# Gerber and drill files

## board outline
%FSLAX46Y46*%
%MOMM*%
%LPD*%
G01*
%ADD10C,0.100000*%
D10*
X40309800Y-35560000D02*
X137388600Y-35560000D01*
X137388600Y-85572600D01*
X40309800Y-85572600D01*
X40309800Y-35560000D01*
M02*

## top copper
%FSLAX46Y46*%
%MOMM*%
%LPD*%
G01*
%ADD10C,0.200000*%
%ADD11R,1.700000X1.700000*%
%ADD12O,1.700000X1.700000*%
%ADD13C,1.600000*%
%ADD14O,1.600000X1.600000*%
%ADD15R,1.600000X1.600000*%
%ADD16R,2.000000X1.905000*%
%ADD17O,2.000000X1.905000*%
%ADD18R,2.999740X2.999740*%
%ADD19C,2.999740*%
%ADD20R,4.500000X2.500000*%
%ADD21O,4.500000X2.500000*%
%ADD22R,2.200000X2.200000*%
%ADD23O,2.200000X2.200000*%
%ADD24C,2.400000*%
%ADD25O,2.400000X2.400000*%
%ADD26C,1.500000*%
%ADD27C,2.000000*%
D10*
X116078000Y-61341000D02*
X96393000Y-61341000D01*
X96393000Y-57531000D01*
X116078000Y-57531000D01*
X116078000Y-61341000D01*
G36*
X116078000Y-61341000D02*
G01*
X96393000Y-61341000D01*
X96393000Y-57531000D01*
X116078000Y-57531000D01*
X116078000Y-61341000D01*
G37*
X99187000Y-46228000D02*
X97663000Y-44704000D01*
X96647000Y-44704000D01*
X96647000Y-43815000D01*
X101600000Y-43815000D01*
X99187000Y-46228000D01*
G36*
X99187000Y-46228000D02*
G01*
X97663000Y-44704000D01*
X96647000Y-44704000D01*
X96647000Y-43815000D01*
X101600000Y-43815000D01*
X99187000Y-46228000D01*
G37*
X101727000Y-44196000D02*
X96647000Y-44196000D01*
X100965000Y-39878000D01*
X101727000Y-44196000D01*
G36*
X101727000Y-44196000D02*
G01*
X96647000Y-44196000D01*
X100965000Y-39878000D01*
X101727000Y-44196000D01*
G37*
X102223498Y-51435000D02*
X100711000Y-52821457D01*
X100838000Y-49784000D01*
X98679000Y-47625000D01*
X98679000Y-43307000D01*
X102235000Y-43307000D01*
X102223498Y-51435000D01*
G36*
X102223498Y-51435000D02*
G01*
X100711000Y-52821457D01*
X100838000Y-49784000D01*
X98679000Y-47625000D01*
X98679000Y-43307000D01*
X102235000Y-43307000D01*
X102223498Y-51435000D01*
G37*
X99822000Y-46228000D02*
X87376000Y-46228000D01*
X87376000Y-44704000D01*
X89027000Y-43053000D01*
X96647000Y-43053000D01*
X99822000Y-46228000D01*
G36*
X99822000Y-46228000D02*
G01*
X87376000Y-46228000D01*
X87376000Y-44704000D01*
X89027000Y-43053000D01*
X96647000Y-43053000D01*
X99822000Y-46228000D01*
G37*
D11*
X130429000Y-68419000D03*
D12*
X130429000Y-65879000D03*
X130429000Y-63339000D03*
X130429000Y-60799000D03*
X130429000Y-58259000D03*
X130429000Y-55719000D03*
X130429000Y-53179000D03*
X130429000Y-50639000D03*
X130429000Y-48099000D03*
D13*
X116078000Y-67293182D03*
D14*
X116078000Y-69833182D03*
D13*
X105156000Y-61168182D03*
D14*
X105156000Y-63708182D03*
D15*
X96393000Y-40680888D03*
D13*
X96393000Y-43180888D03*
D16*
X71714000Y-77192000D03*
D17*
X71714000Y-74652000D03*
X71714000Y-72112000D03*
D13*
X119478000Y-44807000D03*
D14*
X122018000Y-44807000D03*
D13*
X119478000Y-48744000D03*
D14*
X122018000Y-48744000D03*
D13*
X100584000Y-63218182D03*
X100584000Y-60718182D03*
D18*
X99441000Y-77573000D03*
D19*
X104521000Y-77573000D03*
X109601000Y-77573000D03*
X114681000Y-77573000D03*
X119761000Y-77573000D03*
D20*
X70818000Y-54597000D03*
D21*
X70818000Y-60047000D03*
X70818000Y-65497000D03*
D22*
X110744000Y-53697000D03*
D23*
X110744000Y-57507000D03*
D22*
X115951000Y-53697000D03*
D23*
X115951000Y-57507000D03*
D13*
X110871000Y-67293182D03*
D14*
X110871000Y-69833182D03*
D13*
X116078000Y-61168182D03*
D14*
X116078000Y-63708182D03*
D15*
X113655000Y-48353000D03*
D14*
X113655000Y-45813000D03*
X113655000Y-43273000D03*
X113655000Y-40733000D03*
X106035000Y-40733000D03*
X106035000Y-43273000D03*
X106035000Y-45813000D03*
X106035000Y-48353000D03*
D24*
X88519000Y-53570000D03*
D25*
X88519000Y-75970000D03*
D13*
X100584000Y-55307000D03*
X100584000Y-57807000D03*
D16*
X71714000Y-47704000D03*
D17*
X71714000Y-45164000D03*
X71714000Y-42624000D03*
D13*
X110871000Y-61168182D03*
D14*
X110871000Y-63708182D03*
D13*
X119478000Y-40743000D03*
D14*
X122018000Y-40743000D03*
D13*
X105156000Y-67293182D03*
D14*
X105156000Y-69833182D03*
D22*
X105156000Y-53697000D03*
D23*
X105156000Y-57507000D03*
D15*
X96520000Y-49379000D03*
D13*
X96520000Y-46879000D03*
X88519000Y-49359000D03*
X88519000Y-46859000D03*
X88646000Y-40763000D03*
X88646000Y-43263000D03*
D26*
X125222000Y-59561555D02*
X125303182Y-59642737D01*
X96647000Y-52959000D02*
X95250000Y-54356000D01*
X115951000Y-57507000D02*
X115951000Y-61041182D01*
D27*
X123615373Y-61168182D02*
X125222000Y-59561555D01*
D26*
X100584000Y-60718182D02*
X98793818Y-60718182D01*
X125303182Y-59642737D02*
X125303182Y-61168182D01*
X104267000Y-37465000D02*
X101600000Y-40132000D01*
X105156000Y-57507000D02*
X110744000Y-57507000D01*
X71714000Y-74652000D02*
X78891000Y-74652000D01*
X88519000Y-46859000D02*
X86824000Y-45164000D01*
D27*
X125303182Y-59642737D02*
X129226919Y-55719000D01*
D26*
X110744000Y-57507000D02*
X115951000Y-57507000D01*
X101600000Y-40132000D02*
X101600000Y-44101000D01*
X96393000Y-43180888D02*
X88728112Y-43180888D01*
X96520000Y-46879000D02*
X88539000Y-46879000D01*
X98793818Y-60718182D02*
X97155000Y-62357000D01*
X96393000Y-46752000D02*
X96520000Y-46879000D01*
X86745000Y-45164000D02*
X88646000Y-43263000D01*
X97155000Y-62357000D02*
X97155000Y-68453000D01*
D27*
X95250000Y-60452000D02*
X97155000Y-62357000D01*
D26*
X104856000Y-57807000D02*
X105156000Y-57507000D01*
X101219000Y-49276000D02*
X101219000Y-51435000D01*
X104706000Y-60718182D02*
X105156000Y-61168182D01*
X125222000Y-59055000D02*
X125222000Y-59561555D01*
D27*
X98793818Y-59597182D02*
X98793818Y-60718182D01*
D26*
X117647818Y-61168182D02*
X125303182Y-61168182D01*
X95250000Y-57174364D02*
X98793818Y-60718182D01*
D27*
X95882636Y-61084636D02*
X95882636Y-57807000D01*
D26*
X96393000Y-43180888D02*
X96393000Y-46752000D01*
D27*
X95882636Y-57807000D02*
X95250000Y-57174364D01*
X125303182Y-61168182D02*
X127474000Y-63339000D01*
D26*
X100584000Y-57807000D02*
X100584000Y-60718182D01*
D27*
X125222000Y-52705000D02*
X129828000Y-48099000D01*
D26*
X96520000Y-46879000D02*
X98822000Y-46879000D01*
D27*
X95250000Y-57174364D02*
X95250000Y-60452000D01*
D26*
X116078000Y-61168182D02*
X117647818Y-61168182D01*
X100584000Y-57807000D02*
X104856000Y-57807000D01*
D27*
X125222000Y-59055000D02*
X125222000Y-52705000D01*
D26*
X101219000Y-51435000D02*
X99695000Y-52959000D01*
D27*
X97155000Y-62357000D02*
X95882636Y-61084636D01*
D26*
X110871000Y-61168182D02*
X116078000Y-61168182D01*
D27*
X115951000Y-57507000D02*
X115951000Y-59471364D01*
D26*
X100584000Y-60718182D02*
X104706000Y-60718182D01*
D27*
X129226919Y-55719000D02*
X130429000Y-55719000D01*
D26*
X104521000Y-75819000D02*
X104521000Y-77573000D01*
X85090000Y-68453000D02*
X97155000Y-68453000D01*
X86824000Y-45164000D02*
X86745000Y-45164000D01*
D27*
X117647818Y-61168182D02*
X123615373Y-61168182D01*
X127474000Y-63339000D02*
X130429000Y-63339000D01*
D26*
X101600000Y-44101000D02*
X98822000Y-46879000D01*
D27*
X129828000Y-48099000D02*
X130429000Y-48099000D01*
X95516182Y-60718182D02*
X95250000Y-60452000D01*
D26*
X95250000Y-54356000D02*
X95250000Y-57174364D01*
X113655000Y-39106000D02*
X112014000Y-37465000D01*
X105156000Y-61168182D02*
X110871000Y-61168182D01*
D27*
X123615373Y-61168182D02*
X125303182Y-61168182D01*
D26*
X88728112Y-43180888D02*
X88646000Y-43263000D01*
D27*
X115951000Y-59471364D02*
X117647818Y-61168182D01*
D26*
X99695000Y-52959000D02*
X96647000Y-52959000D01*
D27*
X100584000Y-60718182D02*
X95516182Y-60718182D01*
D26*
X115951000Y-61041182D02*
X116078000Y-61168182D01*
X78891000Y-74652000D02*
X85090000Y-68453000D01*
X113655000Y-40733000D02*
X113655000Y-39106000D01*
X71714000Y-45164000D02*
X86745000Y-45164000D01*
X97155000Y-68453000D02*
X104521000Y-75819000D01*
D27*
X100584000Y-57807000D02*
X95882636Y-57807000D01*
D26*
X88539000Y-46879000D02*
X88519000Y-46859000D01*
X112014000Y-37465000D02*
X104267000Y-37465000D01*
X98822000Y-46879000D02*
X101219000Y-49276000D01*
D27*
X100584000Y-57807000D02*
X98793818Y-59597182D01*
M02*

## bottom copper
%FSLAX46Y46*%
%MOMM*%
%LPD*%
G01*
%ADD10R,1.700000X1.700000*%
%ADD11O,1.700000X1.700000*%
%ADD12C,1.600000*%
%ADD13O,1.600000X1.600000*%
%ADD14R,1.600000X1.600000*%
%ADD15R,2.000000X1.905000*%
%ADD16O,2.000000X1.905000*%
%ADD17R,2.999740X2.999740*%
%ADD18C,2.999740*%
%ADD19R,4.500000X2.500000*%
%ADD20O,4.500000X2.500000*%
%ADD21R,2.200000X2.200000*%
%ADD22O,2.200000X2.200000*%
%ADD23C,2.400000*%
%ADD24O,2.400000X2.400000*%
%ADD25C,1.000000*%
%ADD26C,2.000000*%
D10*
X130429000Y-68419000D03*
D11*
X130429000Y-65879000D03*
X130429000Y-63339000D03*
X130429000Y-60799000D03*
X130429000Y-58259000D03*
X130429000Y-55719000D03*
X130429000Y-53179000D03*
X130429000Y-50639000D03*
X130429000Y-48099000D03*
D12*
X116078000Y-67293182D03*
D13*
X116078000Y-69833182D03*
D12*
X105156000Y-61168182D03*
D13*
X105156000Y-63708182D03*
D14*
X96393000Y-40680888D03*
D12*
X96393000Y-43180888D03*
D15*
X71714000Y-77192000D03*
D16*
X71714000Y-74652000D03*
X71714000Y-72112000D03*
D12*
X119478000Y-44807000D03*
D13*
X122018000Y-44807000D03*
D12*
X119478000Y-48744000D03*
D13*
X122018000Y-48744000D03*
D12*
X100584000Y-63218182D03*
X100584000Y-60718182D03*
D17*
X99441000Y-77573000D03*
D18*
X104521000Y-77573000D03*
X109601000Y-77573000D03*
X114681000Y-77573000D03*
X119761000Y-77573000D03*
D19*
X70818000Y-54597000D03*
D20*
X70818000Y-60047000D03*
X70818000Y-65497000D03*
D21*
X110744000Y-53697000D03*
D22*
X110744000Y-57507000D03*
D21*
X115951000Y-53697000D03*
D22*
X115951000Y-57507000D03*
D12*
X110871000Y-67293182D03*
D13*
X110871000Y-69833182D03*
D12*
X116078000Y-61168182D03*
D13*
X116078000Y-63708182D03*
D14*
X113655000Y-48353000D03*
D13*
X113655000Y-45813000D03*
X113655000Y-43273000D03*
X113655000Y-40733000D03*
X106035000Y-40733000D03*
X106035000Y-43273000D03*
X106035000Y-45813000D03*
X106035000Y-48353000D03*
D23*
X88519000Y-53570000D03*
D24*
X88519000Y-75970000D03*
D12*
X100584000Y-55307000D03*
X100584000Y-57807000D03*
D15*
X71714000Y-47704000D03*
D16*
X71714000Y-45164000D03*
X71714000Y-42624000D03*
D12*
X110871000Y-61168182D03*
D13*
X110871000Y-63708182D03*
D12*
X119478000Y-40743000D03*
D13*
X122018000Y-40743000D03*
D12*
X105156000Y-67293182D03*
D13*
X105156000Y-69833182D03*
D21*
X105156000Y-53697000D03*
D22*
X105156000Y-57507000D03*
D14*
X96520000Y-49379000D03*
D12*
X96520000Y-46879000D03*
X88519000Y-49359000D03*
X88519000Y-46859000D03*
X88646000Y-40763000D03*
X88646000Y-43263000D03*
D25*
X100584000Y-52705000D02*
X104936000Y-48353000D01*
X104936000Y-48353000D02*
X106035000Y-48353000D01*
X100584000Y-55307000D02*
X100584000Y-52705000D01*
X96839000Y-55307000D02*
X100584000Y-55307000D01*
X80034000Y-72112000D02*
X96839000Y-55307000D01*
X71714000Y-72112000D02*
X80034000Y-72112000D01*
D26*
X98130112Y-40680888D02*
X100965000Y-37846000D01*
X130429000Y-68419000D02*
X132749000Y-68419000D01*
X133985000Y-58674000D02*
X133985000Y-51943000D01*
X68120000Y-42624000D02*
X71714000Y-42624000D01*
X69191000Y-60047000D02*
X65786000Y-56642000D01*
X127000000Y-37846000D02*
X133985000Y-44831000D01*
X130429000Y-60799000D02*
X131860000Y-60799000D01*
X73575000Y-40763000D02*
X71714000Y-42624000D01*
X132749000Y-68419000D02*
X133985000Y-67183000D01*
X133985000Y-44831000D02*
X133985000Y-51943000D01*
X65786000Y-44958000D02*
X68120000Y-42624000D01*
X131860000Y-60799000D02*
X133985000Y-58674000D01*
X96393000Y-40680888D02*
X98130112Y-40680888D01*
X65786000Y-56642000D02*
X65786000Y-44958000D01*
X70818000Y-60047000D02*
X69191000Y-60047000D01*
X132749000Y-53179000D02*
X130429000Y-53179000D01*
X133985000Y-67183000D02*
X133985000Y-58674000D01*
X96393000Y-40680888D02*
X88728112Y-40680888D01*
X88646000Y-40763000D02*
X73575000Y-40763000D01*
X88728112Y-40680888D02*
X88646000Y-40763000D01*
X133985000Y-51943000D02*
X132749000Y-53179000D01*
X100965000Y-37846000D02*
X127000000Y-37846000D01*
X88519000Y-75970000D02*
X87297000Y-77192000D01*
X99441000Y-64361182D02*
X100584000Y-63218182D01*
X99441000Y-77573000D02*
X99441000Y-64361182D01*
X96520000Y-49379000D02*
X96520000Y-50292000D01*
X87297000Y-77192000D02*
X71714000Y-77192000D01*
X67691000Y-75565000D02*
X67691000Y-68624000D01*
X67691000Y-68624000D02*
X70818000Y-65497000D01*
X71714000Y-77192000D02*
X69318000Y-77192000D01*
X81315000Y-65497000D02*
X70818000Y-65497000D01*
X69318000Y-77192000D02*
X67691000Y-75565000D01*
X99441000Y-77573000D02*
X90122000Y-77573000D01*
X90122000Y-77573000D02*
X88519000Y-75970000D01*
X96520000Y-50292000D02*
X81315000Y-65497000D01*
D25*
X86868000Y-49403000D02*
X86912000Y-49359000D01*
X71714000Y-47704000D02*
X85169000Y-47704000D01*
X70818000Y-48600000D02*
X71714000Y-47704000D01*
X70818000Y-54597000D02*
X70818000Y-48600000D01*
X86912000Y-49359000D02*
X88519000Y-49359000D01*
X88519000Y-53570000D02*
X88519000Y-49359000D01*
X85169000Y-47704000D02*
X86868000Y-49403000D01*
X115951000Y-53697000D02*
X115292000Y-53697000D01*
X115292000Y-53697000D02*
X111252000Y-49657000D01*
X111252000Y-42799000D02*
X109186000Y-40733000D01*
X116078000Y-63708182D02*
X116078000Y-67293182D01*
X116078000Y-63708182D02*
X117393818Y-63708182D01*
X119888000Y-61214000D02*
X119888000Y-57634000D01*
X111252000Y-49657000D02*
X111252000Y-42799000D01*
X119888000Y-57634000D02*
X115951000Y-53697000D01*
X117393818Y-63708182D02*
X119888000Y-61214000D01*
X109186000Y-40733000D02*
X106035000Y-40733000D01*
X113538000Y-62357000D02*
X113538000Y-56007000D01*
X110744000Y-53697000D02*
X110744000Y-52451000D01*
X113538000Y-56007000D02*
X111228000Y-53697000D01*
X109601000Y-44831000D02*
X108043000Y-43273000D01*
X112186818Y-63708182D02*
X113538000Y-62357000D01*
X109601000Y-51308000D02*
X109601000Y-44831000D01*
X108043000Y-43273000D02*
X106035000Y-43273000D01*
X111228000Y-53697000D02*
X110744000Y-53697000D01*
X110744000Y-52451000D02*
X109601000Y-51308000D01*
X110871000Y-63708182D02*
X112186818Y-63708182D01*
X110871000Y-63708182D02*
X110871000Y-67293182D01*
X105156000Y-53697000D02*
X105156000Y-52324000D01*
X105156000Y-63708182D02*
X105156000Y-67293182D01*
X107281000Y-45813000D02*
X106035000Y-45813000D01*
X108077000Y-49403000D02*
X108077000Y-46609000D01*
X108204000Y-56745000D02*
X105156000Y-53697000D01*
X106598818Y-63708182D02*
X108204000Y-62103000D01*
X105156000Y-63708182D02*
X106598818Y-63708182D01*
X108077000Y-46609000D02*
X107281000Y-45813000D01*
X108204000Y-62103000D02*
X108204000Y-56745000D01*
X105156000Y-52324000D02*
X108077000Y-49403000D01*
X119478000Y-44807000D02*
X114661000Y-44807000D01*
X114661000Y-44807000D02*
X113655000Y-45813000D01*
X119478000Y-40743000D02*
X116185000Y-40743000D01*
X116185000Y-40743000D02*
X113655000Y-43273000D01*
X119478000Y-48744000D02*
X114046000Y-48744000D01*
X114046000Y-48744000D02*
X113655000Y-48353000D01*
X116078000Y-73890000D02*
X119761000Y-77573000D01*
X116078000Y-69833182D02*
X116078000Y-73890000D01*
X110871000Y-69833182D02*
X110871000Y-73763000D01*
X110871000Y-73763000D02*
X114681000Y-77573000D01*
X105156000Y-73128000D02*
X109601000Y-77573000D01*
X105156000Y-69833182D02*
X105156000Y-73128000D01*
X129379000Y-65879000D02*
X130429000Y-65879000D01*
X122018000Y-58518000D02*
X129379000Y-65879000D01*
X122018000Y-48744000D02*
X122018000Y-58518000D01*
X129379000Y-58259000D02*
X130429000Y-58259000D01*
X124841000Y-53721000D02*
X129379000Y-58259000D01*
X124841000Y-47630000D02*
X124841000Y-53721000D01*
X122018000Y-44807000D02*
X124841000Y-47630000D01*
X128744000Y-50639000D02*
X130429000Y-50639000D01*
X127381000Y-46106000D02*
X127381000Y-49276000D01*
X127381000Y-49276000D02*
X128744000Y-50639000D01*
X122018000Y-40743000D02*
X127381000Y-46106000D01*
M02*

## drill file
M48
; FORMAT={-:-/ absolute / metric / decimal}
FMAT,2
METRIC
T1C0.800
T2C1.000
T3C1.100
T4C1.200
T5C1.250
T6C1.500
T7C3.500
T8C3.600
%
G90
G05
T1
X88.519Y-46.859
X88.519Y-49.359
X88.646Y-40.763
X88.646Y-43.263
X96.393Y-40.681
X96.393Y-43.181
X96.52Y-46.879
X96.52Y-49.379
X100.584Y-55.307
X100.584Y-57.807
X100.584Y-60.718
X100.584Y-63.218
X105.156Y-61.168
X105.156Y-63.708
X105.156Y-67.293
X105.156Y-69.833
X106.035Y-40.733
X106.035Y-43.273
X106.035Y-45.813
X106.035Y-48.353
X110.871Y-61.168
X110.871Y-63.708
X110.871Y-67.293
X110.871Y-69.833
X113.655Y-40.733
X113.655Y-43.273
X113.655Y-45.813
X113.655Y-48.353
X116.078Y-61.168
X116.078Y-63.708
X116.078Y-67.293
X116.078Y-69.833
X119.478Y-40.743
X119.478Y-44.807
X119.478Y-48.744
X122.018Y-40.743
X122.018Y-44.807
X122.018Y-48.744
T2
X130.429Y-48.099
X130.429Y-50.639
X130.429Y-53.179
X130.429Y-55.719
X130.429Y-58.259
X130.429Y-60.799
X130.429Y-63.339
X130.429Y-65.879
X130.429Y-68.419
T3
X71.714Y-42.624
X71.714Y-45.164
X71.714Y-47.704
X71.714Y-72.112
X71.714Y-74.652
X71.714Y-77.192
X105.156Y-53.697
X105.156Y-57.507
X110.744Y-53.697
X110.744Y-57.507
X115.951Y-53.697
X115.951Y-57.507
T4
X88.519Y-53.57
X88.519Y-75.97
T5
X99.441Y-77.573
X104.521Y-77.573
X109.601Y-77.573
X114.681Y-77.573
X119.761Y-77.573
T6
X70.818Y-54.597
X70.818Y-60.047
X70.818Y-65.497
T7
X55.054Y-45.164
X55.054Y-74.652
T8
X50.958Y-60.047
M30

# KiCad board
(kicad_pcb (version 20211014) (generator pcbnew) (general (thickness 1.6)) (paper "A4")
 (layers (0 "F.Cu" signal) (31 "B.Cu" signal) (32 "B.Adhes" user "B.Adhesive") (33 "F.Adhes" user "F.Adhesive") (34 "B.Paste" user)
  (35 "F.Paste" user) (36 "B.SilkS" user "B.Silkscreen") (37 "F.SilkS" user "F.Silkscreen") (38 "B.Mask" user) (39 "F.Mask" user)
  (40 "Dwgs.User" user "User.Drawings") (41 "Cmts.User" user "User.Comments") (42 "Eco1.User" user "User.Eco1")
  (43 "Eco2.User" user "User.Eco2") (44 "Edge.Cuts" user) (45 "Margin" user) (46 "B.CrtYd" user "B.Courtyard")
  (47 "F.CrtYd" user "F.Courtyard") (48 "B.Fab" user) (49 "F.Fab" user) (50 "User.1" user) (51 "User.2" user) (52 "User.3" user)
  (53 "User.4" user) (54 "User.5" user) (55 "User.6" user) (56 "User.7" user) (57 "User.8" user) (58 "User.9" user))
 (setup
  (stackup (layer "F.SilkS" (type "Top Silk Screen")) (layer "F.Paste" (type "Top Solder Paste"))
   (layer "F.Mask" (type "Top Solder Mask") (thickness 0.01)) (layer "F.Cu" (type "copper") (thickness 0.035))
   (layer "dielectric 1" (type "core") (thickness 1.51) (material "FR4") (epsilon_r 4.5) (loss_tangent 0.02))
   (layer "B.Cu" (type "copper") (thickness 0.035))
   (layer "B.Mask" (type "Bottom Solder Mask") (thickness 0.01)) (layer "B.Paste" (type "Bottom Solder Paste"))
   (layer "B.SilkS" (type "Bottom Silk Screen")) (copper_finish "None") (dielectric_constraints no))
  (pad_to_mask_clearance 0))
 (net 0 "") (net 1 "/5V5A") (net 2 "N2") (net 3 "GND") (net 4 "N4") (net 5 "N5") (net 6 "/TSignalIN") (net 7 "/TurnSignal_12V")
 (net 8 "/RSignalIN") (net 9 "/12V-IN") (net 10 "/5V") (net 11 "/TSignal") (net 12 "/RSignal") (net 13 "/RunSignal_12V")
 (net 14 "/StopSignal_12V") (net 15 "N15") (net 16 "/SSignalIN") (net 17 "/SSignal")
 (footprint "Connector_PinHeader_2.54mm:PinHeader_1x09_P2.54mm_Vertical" (layer "F.Cu") (at 130.429 68.419 180)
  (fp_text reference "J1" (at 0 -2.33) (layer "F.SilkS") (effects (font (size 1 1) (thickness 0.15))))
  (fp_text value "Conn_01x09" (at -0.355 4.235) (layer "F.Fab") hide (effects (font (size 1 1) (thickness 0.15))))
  (pad "1" thru_hole rect (at 0 0 180) (size 1.7 1.7) (drill 1) (layers *.Cu *.Mask) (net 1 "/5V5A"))
  (pad "2" thru_hole oval (at 0 2.54 180) (size 1.7 1.7) (drill 1) (layers *.Cu *.Mask) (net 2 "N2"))
  (pad "3" thru_hole oval (at 0 5.08 180) (size 1.7 1.7) (drill 1) (layers *.Cu *.Mask) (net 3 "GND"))
  (pad "4" thru_hole oval (at 0 7.62 180) (size 1.7 1.7) (drill 1) (layers *.Cu *.Mask) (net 1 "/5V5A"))
  (pad "5" thru_hole oval (at 0 10.16 180) (size 1.7 1.7) (drill 1) (layers *.Cu *.Mask) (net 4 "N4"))
  (pad "6" thru_hole oval (at 0 12.7 180) (size 1.7 1.7) (drill 1) (layers *.Cu *.Mask) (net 3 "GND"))
  (pad "7" thru_hole oval (at 0 15.24 180) (size 1.7 1.7) (drill 1) (layers *.Cu *.Mask) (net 1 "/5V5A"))
  (pad "8" thru_hole oval (at 0 17.78 180) (size 1.7 1.7) (drill 1) (layers *.Cu *.Mask) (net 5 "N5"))
  (pad "9" thru_hole oval (at 0 20.32 180) (size 1.7 1.7) (drill 1) (layers *.Cu *.Mask) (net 3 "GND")))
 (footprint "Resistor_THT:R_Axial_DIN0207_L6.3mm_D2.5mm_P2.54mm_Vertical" (layer "F.Cu") (at 116.078 67.293182 -90)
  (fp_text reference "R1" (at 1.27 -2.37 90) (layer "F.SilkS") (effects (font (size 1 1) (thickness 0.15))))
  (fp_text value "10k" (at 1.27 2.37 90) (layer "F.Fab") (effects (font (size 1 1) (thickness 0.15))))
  (pad "1" thru_hole circle (at 0 0 270) (size 1.6 1.6) (drill 0.8) (layers *.Cu *.Mask) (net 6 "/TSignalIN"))
  (pad "2" thru_hole oval (at 2.54 0 270) (size 1.6 1.6) (drill 0.8) (layers *.Cu *.Mask) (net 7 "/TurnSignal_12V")))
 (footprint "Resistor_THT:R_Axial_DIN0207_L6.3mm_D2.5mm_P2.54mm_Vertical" (layer "F.Cu") (at 105.156 61.168182 -90)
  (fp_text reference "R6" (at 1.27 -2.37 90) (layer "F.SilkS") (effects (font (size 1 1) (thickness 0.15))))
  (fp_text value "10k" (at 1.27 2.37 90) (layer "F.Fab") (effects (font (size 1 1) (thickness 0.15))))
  (pad "1" thru_hole circle (at 0 0 270) (size 1.6 1.6) (drill 0.8) (layers *.Cu *.Mask) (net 3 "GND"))
  (pad "2" thru_hole oval (at 2.54 0 270) (size 1.6 1.6) (drill 0.8) (layers *.Cu *.Mask) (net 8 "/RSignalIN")))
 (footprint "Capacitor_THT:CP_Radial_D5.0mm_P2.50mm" (layer "F.Cu") (at 96.393 40.680888 -90)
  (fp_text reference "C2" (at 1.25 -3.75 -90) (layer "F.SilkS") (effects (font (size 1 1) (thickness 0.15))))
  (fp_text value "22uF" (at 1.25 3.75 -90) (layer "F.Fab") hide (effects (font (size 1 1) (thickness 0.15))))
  (pad "1" thru_hole rect (at 0 0 270) (size 1.6 1.6) (drill 0.8) (layers *.Cu *.Mask) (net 1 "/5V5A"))
  (pad "2" thru_hole circle (at 2.5 0 270) (size 1.6 1.6) (drill 0.8) (layers *.Cu *.Mask) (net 3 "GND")))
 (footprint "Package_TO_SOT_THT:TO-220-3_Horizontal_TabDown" (layer "F.Cu") (at 71.714 77.192 90)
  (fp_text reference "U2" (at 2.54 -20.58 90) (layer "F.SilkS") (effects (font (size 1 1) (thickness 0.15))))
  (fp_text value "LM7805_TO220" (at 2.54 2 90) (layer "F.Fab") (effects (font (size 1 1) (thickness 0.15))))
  (pad "" np_thru_hole oval (at 2.54 -16.66 90) (size 3.5 3.5) (drill 3.5) (layers *.Cu *.Mask))
  (pad "1" thru_hole rect (at 0 0 90) (size 1.905 2) (drill 1.1) (layers *.Cu *.Mask) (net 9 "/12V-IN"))
  (pad "2" thru_hole oval (at 2.54 0 90) (size 1.905 2) (drill 1.1) (layers *.Cu *.Mask) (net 3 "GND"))
  (pad "3" thru_hole oval (at 5.08 0 90) (size 1.905 2) (drill 1.1) (layers *.Cu *.Mask) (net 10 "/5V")))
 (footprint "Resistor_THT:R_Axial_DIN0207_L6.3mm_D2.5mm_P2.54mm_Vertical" (layer "F.Cu") (at 119.478 44.807)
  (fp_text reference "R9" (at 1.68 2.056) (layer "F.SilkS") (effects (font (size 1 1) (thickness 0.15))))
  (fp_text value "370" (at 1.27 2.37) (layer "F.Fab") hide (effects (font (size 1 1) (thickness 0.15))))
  (pad "1" thru_hole circle (at 0 0) (size 1.6 1.6) (drill 0.8) (layers *.Cu *.Mask) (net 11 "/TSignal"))
  (pad "2" thru_hole oval (at 2.54 0) (size 1.6 1.6) (drill 0.8) (layers *.Cu *.Mask) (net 4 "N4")))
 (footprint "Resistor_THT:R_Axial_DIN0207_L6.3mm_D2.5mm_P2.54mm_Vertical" (layer "F.Cu") (at 119.478 48.744)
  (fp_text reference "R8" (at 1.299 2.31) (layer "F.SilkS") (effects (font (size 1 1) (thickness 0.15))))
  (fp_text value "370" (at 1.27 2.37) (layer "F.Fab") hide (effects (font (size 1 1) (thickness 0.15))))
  (pad "1" thru_hole circle (at 0 0) (size 1.6 1.6) (drill 0.8) (layers *.Cu *.Mask) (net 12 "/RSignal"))
  (pad "2" thru_hole oval (at 2.54 0) (size 1.6 1.6) (drill 0.8) (layers *.Cu *.Mask) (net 2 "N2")))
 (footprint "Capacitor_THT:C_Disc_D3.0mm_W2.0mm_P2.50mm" (layer "F.Cu") (at 100.584 63.218182 90)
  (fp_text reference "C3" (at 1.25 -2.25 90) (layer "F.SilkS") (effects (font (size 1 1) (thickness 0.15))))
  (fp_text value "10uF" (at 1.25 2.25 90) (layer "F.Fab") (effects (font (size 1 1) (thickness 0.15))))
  (pad "1" thru_hole circle (at 0 0 90) (size 1.6 1.6) (drill 0.8) (layers *.Cu *.Mask) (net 9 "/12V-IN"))
  (pad "2" thru_hole circle (at 2.5 0 90) (size 1.6 1.6) (drill 0.8) (layers *.Cu *.Mask) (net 3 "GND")))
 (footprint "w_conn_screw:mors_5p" (layer "F.Cu") (at 109.601 77.573)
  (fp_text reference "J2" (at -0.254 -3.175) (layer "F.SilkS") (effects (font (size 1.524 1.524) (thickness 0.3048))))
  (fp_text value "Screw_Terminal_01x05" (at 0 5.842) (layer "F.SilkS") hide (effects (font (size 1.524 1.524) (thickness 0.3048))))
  (pad "1" thru_hole rect locked (at -10.16 0) (size 2.99974 2.99974) (drill 1.24968) (layers *.Cu *.Mask "F.SilkS") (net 9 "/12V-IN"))
  (pad "2" thru_hole circle locked (at -5.08 0) (size 2.99974 2.99974) (drill 1.24968) (layers *.Cu *.Mask "F.SilkS") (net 3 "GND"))
  (pad "3" thru_hole circle locked (at 0 0) (size 2.99974 2.99974) (drill 1.24968) (layers *.Cu *.Mask "F.SilkS") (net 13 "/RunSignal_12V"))
  (pad "4" thru_hole circle locked (at 5.08 0) (size 2.99974 2.99974) (drill 1.24968) (layers *.Cu *.Mask "F.SilkS")
   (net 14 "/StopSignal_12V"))
  (pad "5" thru_hole circle locked (at 10.16 0) (size 2.99974 2.99974) (drill 1.24968) (layers *.Cu *.Mask "F.SilkS")
   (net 7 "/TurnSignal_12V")))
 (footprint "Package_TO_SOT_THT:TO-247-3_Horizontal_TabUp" (layer "F.Cu") (at 70.818 54.597 -90)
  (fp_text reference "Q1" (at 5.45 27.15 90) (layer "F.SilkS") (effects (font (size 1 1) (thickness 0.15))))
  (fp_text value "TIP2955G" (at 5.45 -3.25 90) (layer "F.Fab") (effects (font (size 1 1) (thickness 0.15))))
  (pad "" np_thru_hole oval (at 5.45 19.86 270) (size 3.6 3.6) (drill 3.6) (layers *.Cu *.Mask))
  (pad "1" thru_hole rect (at 0 0 270) (size 2.5 4.5) (drill 1.5) (layers *.Cu *.Mask) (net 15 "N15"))
  (pad "2" thru_hole oval (at 5.45 0 270) (size 2.5 4.5) (drill 1.5) (layers *.Cu *.Mask) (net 1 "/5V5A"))
  (pad "3" thru_hole oval (at 10.9 0 270) (size 2.5 4.5) (drill 1.5) (layers *.Cu *.Mask) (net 9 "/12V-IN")))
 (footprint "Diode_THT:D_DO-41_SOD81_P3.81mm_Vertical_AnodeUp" (layer "F.Cu") (at 110.744 53.697 -90)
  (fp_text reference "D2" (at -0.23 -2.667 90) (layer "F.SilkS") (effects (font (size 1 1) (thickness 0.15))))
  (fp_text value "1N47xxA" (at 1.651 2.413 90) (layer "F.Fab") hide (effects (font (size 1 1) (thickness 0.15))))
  (pad "1" thru_hole rect (at 0 0 270) (size 2.2 2.2) (drill 1.1) (layers *.Cu *.Mask) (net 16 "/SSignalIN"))
  (pad "2" thru_hole oval (at 3.81 0 270) (size 2.2 2.2) (drill 1.1) (layers *.Cu *.Mask) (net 3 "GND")))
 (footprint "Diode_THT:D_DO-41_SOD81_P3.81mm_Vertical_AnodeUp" (layer "F.Cu") (at 115.951 53.697 -90)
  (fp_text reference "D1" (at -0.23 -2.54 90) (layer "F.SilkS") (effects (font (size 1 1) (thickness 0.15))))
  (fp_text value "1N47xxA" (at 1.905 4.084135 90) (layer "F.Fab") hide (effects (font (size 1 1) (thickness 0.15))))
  (pad "1" thru_hole rect (at 0 0 270) (size 2.2 2.2) (drill 1.1) (layers *.Cu *.Mask) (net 6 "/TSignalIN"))
  (pad "2" thru_hole oval (at 3.81 0 270) (size 2.2 2.2) (drill 1.1) (layers *.Cu *.Mask) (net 3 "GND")))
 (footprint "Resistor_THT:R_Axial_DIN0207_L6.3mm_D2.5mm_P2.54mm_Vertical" (layer "F.Cu") (at 110.871 67.293182 -90)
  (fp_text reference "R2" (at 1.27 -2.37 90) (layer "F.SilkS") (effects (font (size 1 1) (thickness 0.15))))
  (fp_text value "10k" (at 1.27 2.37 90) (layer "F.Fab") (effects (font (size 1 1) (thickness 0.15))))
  (pad "1" thru_hole circle (at 0 0 270) (size 1.6 1.6) (drill 0.8) (layers *.Cu *.Mask) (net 16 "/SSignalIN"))
  (pad "2" thru_hole oval (at 2.54 0 270) (size 1.6 1.6) (drill 0.8) (layers *.Cu *.Mask) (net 14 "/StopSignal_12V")))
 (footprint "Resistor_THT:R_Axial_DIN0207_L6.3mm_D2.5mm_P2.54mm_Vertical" (layer "F.Cu") (at 116.078 61.168182 -90)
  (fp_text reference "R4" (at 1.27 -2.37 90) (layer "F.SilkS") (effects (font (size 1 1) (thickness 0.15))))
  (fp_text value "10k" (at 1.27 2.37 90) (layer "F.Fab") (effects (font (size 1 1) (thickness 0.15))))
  (pad "1" thru_hole circle (at 0 0 270) (size 1.6 1.6) (drill 0.8) (layers *.Cu *.Mask) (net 3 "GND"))
  (pad "2" thru_hole oval (at 2.54 0 270) (size 1.6 1.6) (drill 0.8) (layers *.Cu *.Mask) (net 6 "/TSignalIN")))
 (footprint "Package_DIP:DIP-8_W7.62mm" (layer "F.Cu") (at 113.655 48.353 180)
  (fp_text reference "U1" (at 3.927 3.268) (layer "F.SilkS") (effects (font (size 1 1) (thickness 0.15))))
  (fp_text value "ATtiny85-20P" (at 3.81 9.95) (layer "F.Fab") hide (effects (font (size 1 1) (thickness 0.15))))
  (pad "1" thru_hole rect (at 0 0 180) (size 1.6 1.6) (drill 0.8) (layers *.Cu *.Mask) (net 12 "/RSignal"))
  (pad "2" thru_hole oval (at 0 2.54 180) (size 1.6 1.6) (drill 0.8) (layers *.Cu *.Mask) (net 11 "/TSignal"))
  (pad "3" thru_hole oval (at 0 5.08 180) (size 1.6 1.6) (drill 0.8) (layers *.Cu *.Mask) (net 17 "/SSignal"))
  (pad "4" thru_hole oval (at 0 7.62 180) (size 1.6 1.6) (drill 0.8) (layers *.Cu *.Mask) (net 3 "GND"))
  (pad "5" thru_hole oval (at 7.62 7.62 180) (size 1.6 1.6) (drill 0.8) (layers *.Cu *.Mask) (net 6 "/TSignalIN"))
  (pad "6" thru_hole oval (at 7.62 5.08 180) (size 1.6 1.6) (drill 0.8) (layers *.Cu *.Mask) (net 16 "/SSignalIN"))
  (pad "7" thru_hole oval (at 7.62 2.54 180) (size 1.6 1.6) (drill 0.8) (layers *.Cu *.Mask) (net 8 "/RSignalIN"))
  (pad "8" thru_hole oval (at 7.62 0 180) (size 1.6 1.6) (drill 0.8) (layers *.Cu *.Mask) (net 10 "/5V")))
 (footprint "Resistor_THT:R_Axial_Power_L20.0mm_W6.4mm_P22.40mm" (layer "F.Cu") (at 88.519 53.57 -90)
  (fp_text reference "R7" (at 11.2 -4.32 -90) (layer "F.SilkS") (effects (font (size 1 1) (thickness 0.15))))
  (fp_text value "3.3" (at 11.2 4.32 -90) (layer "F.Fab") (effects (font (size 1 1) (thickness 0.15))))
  (pad "1" thru_hole circle (at 0 0 270) (size 2.4 2.4) (drill 1.2) (layers *.Cu *.Mask) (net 15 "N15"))
  (pad "2" thru_hole oval (at 22.4 0 270) (size 2.4 2.4) (drill 1.2) (layers *.Cu *.Mask) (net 9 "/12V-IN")))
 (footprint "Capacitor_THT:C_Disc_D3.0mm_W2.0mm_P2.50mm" (layer "F.Cu") (at 100.584 55.307 -90)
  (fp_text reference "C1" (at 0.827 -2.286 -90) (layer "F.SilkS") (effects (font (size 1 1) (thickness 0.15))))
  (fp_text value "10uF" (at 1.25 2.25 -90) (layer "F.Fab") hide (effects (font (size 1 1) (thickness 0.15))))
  (pad "1" thru_hole circle (at 0 0 270) (size 1.6 1.6) (drill 0.8) (layers *.Cu *.Mask) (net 10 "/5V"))
  (pad "2" thru_hole circle (at 2.5 0 270) (size 1.6 1.6) (drill 0.8) (layers *.Cu *.Mask) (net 3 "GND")))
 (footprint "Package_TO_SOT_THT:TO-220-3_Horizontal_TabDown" (layer "F.Cu") (at 71.714 47.704 90)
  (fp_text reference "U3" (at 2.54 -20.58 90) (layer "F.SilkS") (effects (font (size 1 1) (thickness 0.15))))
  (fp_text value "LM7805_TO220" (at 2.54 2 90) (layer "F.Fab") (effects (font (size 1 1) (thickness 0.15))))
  (pad "" np_thru_hole oval (at 2.54 -16.66 90) (size 3.5 3.5) (drill 3.5) (layers *.Cu *.Mask))
  (pad "1" thru_hole rect (at 0 0 90) (size 1.905 2) (drill 1.1) (layers *.Cu *.Mask) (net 15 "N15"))
  (pad "2" thru_hole oval (at 2.54 0 90) (size 1.905 2) (drill 1.1) (layers *.Cu *.Mask) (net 3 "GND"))
  (pad "3" thru_hole oval (at 5.08 0 90) (size 1.905 2) (drill 1.1) (layers *.Cu *.Mask) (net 1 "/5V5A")))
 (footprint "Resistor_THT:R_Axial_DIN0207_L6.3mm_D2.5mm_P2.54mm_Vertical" (layer "F.Cu") (at 110.871 61.168182 -90)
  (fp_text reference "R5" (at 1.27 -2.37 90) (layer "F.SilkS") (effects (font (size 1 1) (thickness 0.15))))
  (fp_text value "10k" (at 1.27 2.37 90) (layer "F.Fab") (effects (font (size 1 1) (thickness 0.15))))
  (pad "1" thru_hole circle (at 0 0 270) (size 1.6 1.6) (drill 0.8) (layers *.Cu *.Mask) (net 3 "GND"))
  (pad "2" thru_hole oval (at 2.54 0 270) (size 1.6 1.6) (drill 0.8) (layers *.Cu *.Mask) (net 16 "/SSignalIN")))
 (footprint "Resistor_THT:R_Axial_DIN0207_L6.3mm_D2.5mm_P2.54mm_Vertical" (layer "F.Cu") (at 119.478 40.743)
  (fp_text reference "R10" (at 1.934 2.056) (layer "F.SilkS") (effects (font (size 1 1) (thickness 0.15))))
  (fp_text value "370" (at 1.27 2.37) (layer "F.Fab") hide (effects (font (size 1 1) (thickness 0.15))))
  (pad "1" thru_hole circle (at 0 0) (size 1.6 1.6) (drill 0.8) (layers *.Cu *.Mask) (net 17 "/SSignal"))
  (pad "2" thru_hole oval (at 2.54 0) (size 1.6 1.6) (drill 0.8) (layers *.Cu *.Mask) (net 5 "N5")))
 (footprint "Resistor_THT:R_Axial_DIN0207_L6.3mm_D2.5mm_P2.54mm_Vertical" (layer "F.Cu") (at 105.156 67.293182 -90)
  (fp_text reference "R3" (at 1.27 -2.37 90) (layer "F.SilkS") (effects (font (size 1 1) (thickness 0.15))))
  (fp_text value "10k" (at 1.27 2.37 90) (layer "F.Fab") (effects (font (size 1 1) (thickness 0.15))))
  (pad "1" thru_hole circle (at 0 0 270) (size 1.6 1.6) (drill 0.8) (layers *.Cu *.Mask) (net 8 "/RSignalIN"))
  (pad "2" thru_hole oval (at 2.54 0 270) (size 1.6 1.6) (drill 0.8) (layers *.Cu *.Mask) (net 13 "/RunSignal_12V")))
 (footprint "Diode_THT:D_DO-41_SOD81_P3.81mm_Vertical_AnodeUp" (layer "F.Cu") (at 105.156 53.697 -90)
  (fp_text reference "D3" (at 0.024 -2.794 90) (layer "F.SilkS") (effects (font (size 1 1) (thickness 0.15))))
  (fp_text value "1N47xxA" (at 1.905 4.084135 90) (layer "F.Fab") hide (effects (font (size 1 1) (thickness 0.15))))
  (pad "1" thru_hole rect (at 0 0 270) (size 2.2 2.2) (drill 1.1) (layers *.Cu *.Mask) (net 8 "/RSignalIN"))
  (pad "2" thru_hole oval (at 3.81 0 270) (size 2.2 2.2) (drill 1.1) (layers *.Cu *.Mask) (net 3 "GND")))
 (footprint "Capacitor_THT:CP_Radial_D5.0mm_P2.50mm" (layer "F.Cu") (at 96.52 49.379 90)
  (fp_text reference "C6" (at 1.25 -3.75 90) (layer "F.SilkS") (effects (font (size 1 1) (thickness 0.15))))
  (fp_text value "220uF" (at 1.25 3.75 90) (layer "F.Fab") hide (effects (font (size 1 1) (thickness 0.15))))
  (pad "1" thru_hole rect (at 0 0 90) (size 1.6 1.6) (drill 0.8) (layers *.Cu *.Mask) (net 9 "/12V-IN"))
  (pad "2" thru_hole circle (at 2.5 0 90) (size 1.6 1.6) (drill 0.8) (layers *.Cu *.Mask) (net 3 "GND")))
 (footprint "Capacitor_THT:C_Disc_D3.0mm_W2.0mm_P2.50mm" (layer "F.Cu") (at 88.519 49.359 90)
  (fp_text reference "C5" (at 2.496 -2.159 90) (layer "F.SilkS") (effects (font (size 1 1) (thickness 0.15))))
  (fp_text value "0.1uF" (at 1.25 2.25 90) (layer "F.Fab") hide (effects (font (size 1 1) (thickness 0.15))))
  (pad "1" thru_hole circle (at 0 0 90) (size 1.6 1.6) (drill 0.8) (layers *.Cu *.Mask) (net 15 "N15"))
  (pad "2" thru_hole circle (at 2.5 0 90) (size 1.6 1.6) (drill 0.8) (layers *.Cu *.Mask) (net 3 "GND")))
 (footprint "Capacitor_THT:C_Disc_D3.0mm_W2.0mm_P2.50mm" (layer "F.Cu") (at 88.646 40.763 -90)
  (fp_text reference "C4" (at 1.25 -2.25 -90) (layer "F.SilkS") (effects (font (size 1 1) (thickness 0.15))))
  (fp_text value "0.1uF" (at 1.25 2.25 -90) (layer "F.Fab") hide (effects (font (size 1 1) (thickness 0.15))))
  (pad "1" thru_hole circle (at 0 0 270) (size 1.6 1.6) (drill 0.8) (layers *.Cu *.Mask) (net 1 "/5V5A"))
  (pad "2" thru_hole circle (at 2.5 0 270) (size 1.6 1.6) (drill 0.8) (layers *.Cu *.Mask) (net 3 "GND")))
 (gr_poly (pts (xy 116.078 61.341) (xy 96.393 61.341) (xy 96.393 57.531) (xy 116.078 57.531)) (layer "F.Cu") (width 0.2) (fill solid))
 (gr_poly
  (pts (xy 99.187 46.228) (xy 97.663 44.704) (xy 96.647 44.704) (xy 96.647 43.815) (xy 101.6 43.815)) (layer "F.Cu") (width 0.2)
  (fill solid))
 (gr_poly (pts (xy 101.727 44.196) (xy 96.647 44.196) (xy 100.965 39.878)) (layer "F.Cu") (width 0.2) (fill solid))
 (gr_poly
  (pts (xy 102.223498 51.435) (xy 100.711 52.821457) (xy 100.838 49.784) (xy 98.679 47.625) (xy 98.679 43.307) (xy 102.235 43.307))
  (layer "F.Cu") (width 0.2) (fill solid))
 (gr_poly
  (pts (xy 99.822 46.228) (xy 87.376 46.228) (xy 87.376 44.704) (xy 89.027 43.053) (xy 96.647 43.053)) (layer "F.Cu") (width 0.2)
  (fill solid))
 (gr_rect (start 40.3098 35.56) (end 137.3886 85.5726) (layer "Edge.Cuts") (width 0.1) (fill none))
 (segment (start 100.584 52.705) (end 104.936 48.353) (width 1) (layer "B.Cu") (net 10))
 (segment (start 104.936 48.353) (end 106.035 48.353) (width 1) (layer "B.Cu") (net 10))
 (segment (start 100.584 55.307) (end 100.584 52.705) (width 1) (layer "B.Cu") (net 10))
 (segment (start 96.839 55.307) (end 100.584 55.307) (width 1) (layer "B.Cu") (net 10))
 (segment (start 80.034 72.112) (end 96.839 55.307) (width 1) (layer "B.Cu") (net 10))
 (segment (start 71.714 72.112) (end 80.034 72.112) (width 1) (layer "B.Cu") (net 10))
 (segment (start 125.222 59.561555) (end 125.303182 59.642737) (width 1.5) (layer "F.Cu") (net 3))
 (segment (start 96.647 52.959) (end 95.25 54.356) (width 1.5) (layer "F.Cu") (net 3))
 (segment (start 115.951 57.507) (end 115.951 61.041182) (width 1.5) (layer "F.Cu") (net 3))
 (segment (start 123.615373 61.168182) (end 125.222 59.561555) (width 2) (layer "F.Cu") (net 3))
 (segment (start 100.584 60.718182) (end 98.793818 60.718182) (width 1.5) (layer "F.Cu") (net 3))
 (segment (start 125.303182 59.642737) (end 125.303182 61.168182) (width 1.5) (layer "F.Cu") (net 3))
 (segment (start 104.267 37.465) (end 101.6 40.132) (width 1.5) (layer "F.Cu") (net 3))
 (segment (start 105.156 57.507) (end 110.744 57.507) (width 1.5) (layer "F.Cu") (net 3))
 (segment (start 71.714 74.652) (end 78.891 74.652) (width 1.5) (layer "F.Cu") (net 3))
 (segment (start 88.519 46.859) (end 86.824 45.164) (width 1.5) (layer "F.Cu") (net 3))
 (segment (start 125.303182 59.642737) (end 129.226919 55.719) (width 2) (layer "F.Cu") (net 3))
 (segment (start 110.744 57.507) (end 115.951 57.507) (width 1.5) (layer "F.Cu") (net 3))
 (segment (start 101.6 40.132) (end 101.6 44.101) (width 1.5) (layer "F.Cu") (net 3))
 (segment (start 96.393 43.180888) (end 88.728112 43.180888) (width 1.5) (layer "F.Cu") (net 3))
 (segment (start 96.52 46.879) (end 88.539 46.879) (width 1.5) (layer "F.Cu") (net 3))
 (segment (start 98.793818 60.718182) (end 97.155 62.357) (width 1.5) (layer "F.Cu") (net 3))
 (segment (start 96.393 46.752) (end 96.52 46.879) (width 1.5) (layer "F.Cu") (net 3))
 (segment (start 86.745 45.164) (end 88.646 43.263) (width 1.5) (layer "F.Cu") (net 3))
 (segment (start 97.155 62.357) (end 97.155 68.453) (width 1.5) (layer "F.Cu") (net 3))
 (segment (start 95.25 60.452) (end 97.155 62.357) (width 2) (layer "F.Cu") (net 3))
 (segment (start 104.856 57.807) (end 105.156 57.507) (width 1.5) (layer "F.Cu") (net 3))
 (segment (start 101.219 49.276) (end 101.219 51.435) (width 1.5) (layer "F.Cu") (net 3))
 (segment (start 104.706 60.718182) (end 105.156 61.168182) (width 1.5) (layer "F.Cu") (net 3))
 (segment (start 125.222 59.055) (end 125.222 59.561555) (width 1.5) (layer "F.Cu") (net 3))
 (segment (start 98.793818 59.597182) (end 98.793818 60.718182) (width 2) (layer "F.Cu") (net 3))
 (segment (start 117.647818 61.168182) (end 125.303182 61.168182) (width 1.5) (layer "F.Cu") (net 3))
 (segment (start 95.25 57.174364) (end 98.793818 60.718182) (width 1.5) (layer "F.Cu") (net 3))
 (segment (start 95.882636 61.084636) (end 95.882636 57.807) (width 2) (layer "F.Cu") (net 3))
 (segment (start 96.393 43.180888) (end 96.393 46.752) (width 1.5) (layer "F.Cu") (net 3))
 (segment (start 95.882636 57.807) (end 95.25 57.174364) (width 2) (layer "F.Cu") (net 3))
 (segment (start 125.303182 61.168182) (end 127.474 63.339) (width 2) (layer "F.Cu") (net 3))
 (segment (start 100.584 57.807) (end 100.584 60.718182) (width 1.5) (layer "F.Cu") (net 3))
 (segment (start 125.222 52.705) (end 129.828 48.099) (width 2) (layer "F.Cu") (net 3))
 (segment (start 96.52 46.879) (end 98.822 46.879) (width 1.5) (layer "F.Cu") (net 3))
 (segment (start 95.25 57.174364) (end 95.25 60.452) (width 2) (layer "F.Cu") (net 3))
 (segment (start 116.078 61.168182) (end 117.647818 61.168182) (width 1.5) (layer "F.Cu") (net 3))
 (segment (start 100.584 57.807) (end 104.856 57.807) (width 1.5) (layer "F.Cu") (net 3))
 (segment (start 125.222 59.055) (end 125.222 52.705) (width 2) (layer "F.Cu") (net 3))
 (segment (start 101.219 51.435) (end 99.695 52.959) (width 1.5) (layer "F.Cu") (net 3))
 (segment (start 97.155 62.357) (end 95.882636 61.084636) (width 2) (layer "F.Cu") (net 3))
 (segment (start 110.871 61.168182) (end 116.078 61.168182) (width 1.5) (layer "F.Cu") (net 3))
 (segment (start 115.951 57.507) (end 115.951 59.471364) (width 2) (layer "F.Cu") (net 3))
 (segment (start 100.584 60.718182) (end 104.706 60.718182) (width 1.5) (layer "F.Cu") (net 3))
 (segment (start 129.226919 55.719) (end 130.429 55.719) (width 2) (layer "F.Cu") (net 3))
 (segment (start 104.521 75.819) (end 104.521 77.573) (width 1.5) (layer "F.Cu") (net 3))
 (segment (start 85.09 68.453) (end 97.155 68.453) (width 1.5) (layer "F.Cu") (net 3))
 (segment (start 86.824 45.164) (end 86.745 45.164) (width 1.5) (layer "F.Cu") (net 3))
 (segment (start 117.647818 61.168182) (end 123.615373 61.168182) (width 2) (layer "F.Cu") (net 3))
 (segment (start 127.474 63.339) (end 130.429 63.339) (width 2) (layer "F.Cu") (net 3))
 (segment (start 101.6 44.101) (end 98.822 46.879) (width 1.5) (layer "F.Cu") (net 3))
 (segment (start 129.828 48.099) (end 130.429 48.099) (width 2) (layer "F.Cu") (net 3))
 (segment (start 95.516182 60.718182) (end 95.25 60.452) (width 2) (layer "F.Cu") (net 3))
 (segment (start 95.25 54.356) (end 95.25 57.174364) (width 1.5) (layer "F.Cu") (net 3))
 (segment (start 113.655 39.106) (end 112.014 37.465) (width 1.5) (layer "F.Cu") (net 3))
 (segment (start 105.156 61.168182) (end 110.871 61.168182) (width 1.5) (layer "F.Cu") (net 3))
 (segment (start 123.615373 61.168182) (end 125.303182 61.168182) (width 2) (layer "F.Cu") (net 3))
 (segment (start 88.728112 43.180888) (end 88.646 43.263) (width 1.5) (layer "F.Cu") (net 3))
 (segment (start 115.951 59.471364) (end 117.647818 61.168182) (width 2) (layer "F.Cu") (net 3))
 (segment (start 99.695 52.959) (end 96.647 52.959) (width 1.5) (layer "F.Cu") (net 3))
 (segment (start 100.584 60.718182) (end 95.516182 60.718182) (width 2) (layer "F.Cu") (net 3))
 (segment (start 115.951 61.041182) (end 116.078 61.168182) (width 1.5) (layer "F.Cu") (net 3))
 (segment (start 78.891 74.652) (end 85.09 68.453) (width 1.5) (layer "F.Cu") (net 3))
 (segment (start 113.655 40.733) (end 113.655 39.106) (width 1.5) (layer "F.Cu") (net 3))
 (segment (start 71.714 45.164) (end 86.745 45.164) (width 1.5) (layer "F.Cu") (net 3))
 (segment (start 97.155 68.453) (end 104.521 75.819) (width 1.5) (layer "F.Cu") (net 3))
 (segment (start 100.584 57.807) (end 95.882636 57.807) (width 2) (layer "F.Cu") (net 3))
 (segment (start 88.539 46.879) (end 88.519 46.859) (width 1.5) (layer "F.Cu") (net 3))
 (segment (start 112.014 37.465) (end 104.267 37.465) (width 1.5) (layer "F.Cu") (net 3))
 (segment (start 98.822 46.879) (end 101.219 49.276) (width 1.5) (layer "F.Cu") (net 3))
 (segment (start 100.584 57.807) (end 98.793818 59.597182) (width 2) (layer "F.Cu") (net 3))
 (segment (start 98.130112 40.680888) (end 100.965 37.846) (width 2) (layer "B.Cu") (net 1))
 (segment (start 130.429 68.419) (end 132.749 68.419) (width 2) (layer "B.Cu") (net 1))
 (segment (start 133.985 58.674) (end 133.985 51.943) (width 2) (layer "B.Cu") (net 1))
 (segment (start 68.12 42.624) (end 71.714 42.624) (width 2) (layer "B.Cu") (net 1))
 (segment (start 69.191 60.047) (end 65.786 56.642) (width 2) (layer "B.Cu") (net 1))
 (segment (start 127 37.846) (end 133.985 44.831) (width 2) (layer "B.Cu") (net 1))
 (segment (start 130.429 60.799) (end 131.86 60.799) (width 2) (layer "B.Cu") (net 1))
 (segment (start 73.575 40.763) (end 71.714 42.624) (width 2) (layer "B.Cu") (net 1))
 (segment (start 132.749 68.419) (end 133.985 67.183) (width 2) (layer "B.Cu") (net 1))
 (segment (start 133.985 44.831) (end 133.985 51.943) (width 2) (layer "B.Cu") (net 1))
 (segment (start 65.786 44.958) (end 68.12 42.624) (width 2) (layer "B.Cu") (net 1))
 (segment (start 131.86 60.799) (end 133.985 58.674) (width 2) (layer "B.Cu") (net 1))
 (segment (start 96.393 40.680888) (end 98.130112 40.680888) (width 2) (layer "B.Cu") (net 1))
 (segment (start 65.786 56.642) (end 65.786 44.958) (width 2) (layer "B.Cu") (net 1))
 (segment (start 70.818 60.047) (end 69.191 60.047) (width 2) (layer "B.Cu") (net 1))
 (segment (start 132.749 53.179) (end 130.429 53.179) (width 2) (layer "B.Cu") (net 1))
 (segment (start 133.985 67.183) (end 133.985 58.674) (width 2) (layer "B.Cu") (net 1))
 (segment (start 96.393 40.680888) (end 88.728112 40.680888) (width 2) (layer "B.Cu") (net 1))
 (segment (start 88.646 40.763) (end 73.575 40.763) (width 2) (layer "B.Cu") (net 1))
 (segment (start 88.728112 40.680888) (end 88.646 40.763) (width 2) (layer "B.Cu") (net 1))
 (segment (start 133.985 51.943) (end 132.749 53.179) (width 2) (layer "B.Cu") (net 1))
 (segment (start 100.965 37.846) (end 127 37.846) (width 2) (layer "B.Cu") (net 1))
 (segment (start 88.519 75.97) (end 87.297 77.192) (width 2) (layer "B.Cu") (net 9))
 (segment (start 99.441 64.361182) (end 100.584 63.218182) (width 2) (layer "B.Cu") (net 9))
 (segment (start 99.441 77.573) (end 99.441 64.361182) (width 2) (layer "B.Cu") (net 9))
 (segment (start 96.52 49.379) (end 96.52 50.292) (width 2) (layer "B.Cu") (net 9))
 (segment (start 87.297 77.192) (end 71.714 77.192) (width 2) (layer "B.Cu") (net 9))
 (segment (start 67.691 75.565) (end 67.691 68.624) (width 2) (layer "B.Cu") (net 9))
 (segment (start 67.691 68.624) (end 70.818 65.497) (width 2) (layer "B.Cu") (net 9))
 (segment (start 71.714 77.192) (end 69.318 77.192) (width 2) (layer "B.Cu") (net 9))
 (segment (start 81.315 65.497) (end 70.818 65.497) (width 2) (layer "B.Cu") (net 9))
 (segment (start 69.318 77.192) (end 67.691 75.565) (width 2) (layer "B.Cu") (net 9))
 (segment (start 99.441 77.573) (end 90.122 77.573) (width 2) (layer "B.Cu") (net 9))
 (segment (start 90.122 77.573) (end 88.519 75.97) (width 2) (layer "B.Cu") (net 9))
 (segment (start 96.52 50.292) (end 81.315 65.497) (width 2) (layer "B.Cu") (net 9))
 (segment (start 86.868 49.403) (end 86.912 49.359) (width 1) (layer "B.Cu") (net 15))
 (segment (start 71.714 47.704) (end 85.169 47.704) (width 1) (layer "B.Cu") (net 15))
 (segment (start 70.818 48.6) (end 71.714 47.704) (width 1) (layer "B.Cu") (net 15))
 (segment (start 70.818 54.597) (end 70.818 48.6) (width 1) (layer "B.Cu") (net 15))
 (segment (start 86.912 49.359) (end 88.519 49.359) (width 1) (layer "B.Cu") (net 15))
 (segment (start 88.519 53.57) (end 88.519 49.359) (width 1) (layer "B.Cu") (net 15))
 (segment (start 85.169 47.704) (end 86.868 49.403) (width 1) (layer "B.Cu") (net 15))
 (segment (start 115.951 53.697) (end 115.292 53.697) (width 1) (layer "B.Cu") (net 6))
 (segment (start 115.292 53.697) (end 111.252 49.657) (width 1) (layer "B.Cu") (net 6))
 (segment (start 111.252 42.799) (end 109.186 40.733) (width 1) (layer "B.Cu") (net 6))
 (segment (start 116.078 63.708182) (end 116.078 67.293182) (width 1) (layer "B.Cu") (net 6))
 (segment (start 116.078 63.708182) (end 117.393818 63.708182) (width 1) (layer "B.Cu") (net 6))
 (segment (start 119.888 61.214) (end 119.888 57.634) (width 1) (layer "B.Cu") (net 6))
 (segment (start 111.252 49.657) (end 111.252 42.799) (width 1) (layer "B.Cu") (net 6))
 (segment (start 119.888 57.634) (end 115.951 53.697) (width 1) (layer "B.Cu") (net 6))
 (segment (start 117.393818 63.708182) (end 119.888 61.214) (width 1) (layer "B.Cu") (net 6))
 (segment (start 109.186 40.733) (end 106.035 40.733) (width 1) (layer "B.Cu") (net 6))
 (segment (start 113.538 62.357) (end 113.538 56.007) (width 1) (layer "B.Cu") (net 16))
 (segment (start 110.744 53.697) (end 110.744 52.451) (width 1) (layer "B.Cu") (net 16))
 (segment (start 113.538 56.007) (end 111.228 53.697) (width 1) (layer "B.Cu") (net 16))
 (segment (start 109.601 44.831) (end 108.043 43.273) (width 1) (layer "B.Cu") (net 16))
 (segment (start 112.186818 63.708182) (end 113.538 62.357) (width 1) (layer "B.Cu") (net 16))
 (segment (start 109.601 51.308) (end 109.601 44.831) (width 1) (layer "B.Cu") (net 16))
 (segment (start 108.043 43.273) (end 106.035 43.273) (width 1) (layer "B.Cu") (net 16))
 (segment (start 111.228 53.697) (end 110.744 53.697) (width 1) (layer "B.Cu") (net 16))
 (segment (start 110.744 52.451) (end 109.601 51.308) (width 1) (layer "B.Cu") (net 16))
 (segment (start 110.871 63.708182) (end 112.186818 63.708182) (width 1) (layer "B.Cu") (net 16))
 (segment (start 110.871 63.708182) (end 110.871 67.293182) (width 1) (layer "B.Cu") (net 16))
 (segment (start 105.156 53.697) (end 105.156 52.324) (width 1) (layer "B.Cu") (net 8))
 (segment (start 105.156 63.708182) (end 105.156 67.293182) (width 1) (layer "B.Cu") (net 8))
 (segment (start 107.281 45.813) (end 106.035 45.813) (width 1) (layer "B.Cu") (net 8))
 (segment (start 108.077 49.403) (end 108.077 46.609) (width 1) (layer "B.Cu") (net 8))
 (segment (start 108.204 56.745) (end 105.156 53.697) (width 1) (layer "B.Cu") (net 8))
 (segment (start 106.598818 63.708182) (end 108.204 62.103) (width 1) (layer "B.Cu") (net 8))
 (segment (start 105.156 63.708182) (end 106.598818 63.708182) (width 1) (layer "B.Cu") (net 8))
 (segment (start 108.077 46.609) (end 107.281 45.813) (width 1) (layer "B.Cu") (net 8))
 (segment (start 108.204 62.103) (end 108.204 56.745) (width 1) (layer "B.Cu") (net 8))
 (segment (start 105.156 52.324) (end 108.077 49.403) (width 1) (layer "B.Cu") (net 8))
 (segment (start 119.478 44.807) (end 114.661 44.807) (width 1) (layer "B.Cu") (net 11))
 (segment (start 114.661 44.807) (end 113.655 45.813) (width 1) (layer "B.Cu") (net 11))
 (segment (start 119.478 40.743) (end 116.185 40.743) (width 1) (layer "B.Cu") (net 17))
 (segment (start 116.185 40.743) (end 113.655 43.273) (width 1) (layer "B.Cu") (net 17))
 (segment (start 119.478 48.744) (end 114.046 48.744) (width 1) (layer "B.Cu") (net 12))
 (segment (start 114.046 48.744) (end 113.655 48.353) (width 1) (layer "B.Cu") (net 12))
 (segment (start 116.078 73.89) (end 119.761 77.573) (width 1) (layer "B.Cu") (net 7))
 (segment (start 116.078 69.833182) (end 116.078 73.89) (width 1) (layer "B.Cu") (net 7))
 (segment (start 110.871 69.833182) (end 110.871 73.763) (width 1) (layer "B.Cu") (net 14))
 (segment (start 110.871 73.763) (end 114.681 77.573) (width 1) (layer "B.Cu") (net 14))
 (segment (start 105.156 73.128) (end 109.601 77.573) (width 1) (layer "B.Cu") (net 13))
 (segment (start 105.156 69.833182) (end 105.156 73.128) (width 1) (layer "B.Cu") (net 13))
 (segment (start 129.379 65.879) (end 130.429 65.879) (width 1) (layer "B.Cu") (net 2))
 (segment (start 122.018 58.518) (end 129.379 65.879) (width 1) (layer "B.Cu") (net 2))
 (segment (start 122.018 48.744) (end 122.018 58.518) (width 1) (layer "B.Cu") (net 2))
 (segment (start 129.379 58.259) (end 130.429 58.259) (width 1) (layer "B.Cu") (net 4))
 (segment (start 124.841 53.721) (end 129.379 58.259) (width 1) (layer "B.Cu") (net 4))
 (segment (start 124.841 47.63) (end 124.841 53.721) (width 1) (layer "B.Cu") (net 4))
 (segment (start 122.018 44.807) (end 124.841 47.63) (width 1) (layer "B.Cu") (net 4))
 (segment (start 128.744 50.639) (end 130.429 50.639) (width 1) (layer "B.Cu") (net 5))
 (segment (start 127.381 46.106) (end 127.381 49.276) (width 1) (layer "B.Cu") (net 5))
 (segment (start 127.381 49.276) (end 128.744 50.639) (width 1) (layer "B.Cu") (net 5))
 (segment (start 122.018 40.743) (end 127.381 46.106) (width 1) (layer "B.Cu") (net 5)))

